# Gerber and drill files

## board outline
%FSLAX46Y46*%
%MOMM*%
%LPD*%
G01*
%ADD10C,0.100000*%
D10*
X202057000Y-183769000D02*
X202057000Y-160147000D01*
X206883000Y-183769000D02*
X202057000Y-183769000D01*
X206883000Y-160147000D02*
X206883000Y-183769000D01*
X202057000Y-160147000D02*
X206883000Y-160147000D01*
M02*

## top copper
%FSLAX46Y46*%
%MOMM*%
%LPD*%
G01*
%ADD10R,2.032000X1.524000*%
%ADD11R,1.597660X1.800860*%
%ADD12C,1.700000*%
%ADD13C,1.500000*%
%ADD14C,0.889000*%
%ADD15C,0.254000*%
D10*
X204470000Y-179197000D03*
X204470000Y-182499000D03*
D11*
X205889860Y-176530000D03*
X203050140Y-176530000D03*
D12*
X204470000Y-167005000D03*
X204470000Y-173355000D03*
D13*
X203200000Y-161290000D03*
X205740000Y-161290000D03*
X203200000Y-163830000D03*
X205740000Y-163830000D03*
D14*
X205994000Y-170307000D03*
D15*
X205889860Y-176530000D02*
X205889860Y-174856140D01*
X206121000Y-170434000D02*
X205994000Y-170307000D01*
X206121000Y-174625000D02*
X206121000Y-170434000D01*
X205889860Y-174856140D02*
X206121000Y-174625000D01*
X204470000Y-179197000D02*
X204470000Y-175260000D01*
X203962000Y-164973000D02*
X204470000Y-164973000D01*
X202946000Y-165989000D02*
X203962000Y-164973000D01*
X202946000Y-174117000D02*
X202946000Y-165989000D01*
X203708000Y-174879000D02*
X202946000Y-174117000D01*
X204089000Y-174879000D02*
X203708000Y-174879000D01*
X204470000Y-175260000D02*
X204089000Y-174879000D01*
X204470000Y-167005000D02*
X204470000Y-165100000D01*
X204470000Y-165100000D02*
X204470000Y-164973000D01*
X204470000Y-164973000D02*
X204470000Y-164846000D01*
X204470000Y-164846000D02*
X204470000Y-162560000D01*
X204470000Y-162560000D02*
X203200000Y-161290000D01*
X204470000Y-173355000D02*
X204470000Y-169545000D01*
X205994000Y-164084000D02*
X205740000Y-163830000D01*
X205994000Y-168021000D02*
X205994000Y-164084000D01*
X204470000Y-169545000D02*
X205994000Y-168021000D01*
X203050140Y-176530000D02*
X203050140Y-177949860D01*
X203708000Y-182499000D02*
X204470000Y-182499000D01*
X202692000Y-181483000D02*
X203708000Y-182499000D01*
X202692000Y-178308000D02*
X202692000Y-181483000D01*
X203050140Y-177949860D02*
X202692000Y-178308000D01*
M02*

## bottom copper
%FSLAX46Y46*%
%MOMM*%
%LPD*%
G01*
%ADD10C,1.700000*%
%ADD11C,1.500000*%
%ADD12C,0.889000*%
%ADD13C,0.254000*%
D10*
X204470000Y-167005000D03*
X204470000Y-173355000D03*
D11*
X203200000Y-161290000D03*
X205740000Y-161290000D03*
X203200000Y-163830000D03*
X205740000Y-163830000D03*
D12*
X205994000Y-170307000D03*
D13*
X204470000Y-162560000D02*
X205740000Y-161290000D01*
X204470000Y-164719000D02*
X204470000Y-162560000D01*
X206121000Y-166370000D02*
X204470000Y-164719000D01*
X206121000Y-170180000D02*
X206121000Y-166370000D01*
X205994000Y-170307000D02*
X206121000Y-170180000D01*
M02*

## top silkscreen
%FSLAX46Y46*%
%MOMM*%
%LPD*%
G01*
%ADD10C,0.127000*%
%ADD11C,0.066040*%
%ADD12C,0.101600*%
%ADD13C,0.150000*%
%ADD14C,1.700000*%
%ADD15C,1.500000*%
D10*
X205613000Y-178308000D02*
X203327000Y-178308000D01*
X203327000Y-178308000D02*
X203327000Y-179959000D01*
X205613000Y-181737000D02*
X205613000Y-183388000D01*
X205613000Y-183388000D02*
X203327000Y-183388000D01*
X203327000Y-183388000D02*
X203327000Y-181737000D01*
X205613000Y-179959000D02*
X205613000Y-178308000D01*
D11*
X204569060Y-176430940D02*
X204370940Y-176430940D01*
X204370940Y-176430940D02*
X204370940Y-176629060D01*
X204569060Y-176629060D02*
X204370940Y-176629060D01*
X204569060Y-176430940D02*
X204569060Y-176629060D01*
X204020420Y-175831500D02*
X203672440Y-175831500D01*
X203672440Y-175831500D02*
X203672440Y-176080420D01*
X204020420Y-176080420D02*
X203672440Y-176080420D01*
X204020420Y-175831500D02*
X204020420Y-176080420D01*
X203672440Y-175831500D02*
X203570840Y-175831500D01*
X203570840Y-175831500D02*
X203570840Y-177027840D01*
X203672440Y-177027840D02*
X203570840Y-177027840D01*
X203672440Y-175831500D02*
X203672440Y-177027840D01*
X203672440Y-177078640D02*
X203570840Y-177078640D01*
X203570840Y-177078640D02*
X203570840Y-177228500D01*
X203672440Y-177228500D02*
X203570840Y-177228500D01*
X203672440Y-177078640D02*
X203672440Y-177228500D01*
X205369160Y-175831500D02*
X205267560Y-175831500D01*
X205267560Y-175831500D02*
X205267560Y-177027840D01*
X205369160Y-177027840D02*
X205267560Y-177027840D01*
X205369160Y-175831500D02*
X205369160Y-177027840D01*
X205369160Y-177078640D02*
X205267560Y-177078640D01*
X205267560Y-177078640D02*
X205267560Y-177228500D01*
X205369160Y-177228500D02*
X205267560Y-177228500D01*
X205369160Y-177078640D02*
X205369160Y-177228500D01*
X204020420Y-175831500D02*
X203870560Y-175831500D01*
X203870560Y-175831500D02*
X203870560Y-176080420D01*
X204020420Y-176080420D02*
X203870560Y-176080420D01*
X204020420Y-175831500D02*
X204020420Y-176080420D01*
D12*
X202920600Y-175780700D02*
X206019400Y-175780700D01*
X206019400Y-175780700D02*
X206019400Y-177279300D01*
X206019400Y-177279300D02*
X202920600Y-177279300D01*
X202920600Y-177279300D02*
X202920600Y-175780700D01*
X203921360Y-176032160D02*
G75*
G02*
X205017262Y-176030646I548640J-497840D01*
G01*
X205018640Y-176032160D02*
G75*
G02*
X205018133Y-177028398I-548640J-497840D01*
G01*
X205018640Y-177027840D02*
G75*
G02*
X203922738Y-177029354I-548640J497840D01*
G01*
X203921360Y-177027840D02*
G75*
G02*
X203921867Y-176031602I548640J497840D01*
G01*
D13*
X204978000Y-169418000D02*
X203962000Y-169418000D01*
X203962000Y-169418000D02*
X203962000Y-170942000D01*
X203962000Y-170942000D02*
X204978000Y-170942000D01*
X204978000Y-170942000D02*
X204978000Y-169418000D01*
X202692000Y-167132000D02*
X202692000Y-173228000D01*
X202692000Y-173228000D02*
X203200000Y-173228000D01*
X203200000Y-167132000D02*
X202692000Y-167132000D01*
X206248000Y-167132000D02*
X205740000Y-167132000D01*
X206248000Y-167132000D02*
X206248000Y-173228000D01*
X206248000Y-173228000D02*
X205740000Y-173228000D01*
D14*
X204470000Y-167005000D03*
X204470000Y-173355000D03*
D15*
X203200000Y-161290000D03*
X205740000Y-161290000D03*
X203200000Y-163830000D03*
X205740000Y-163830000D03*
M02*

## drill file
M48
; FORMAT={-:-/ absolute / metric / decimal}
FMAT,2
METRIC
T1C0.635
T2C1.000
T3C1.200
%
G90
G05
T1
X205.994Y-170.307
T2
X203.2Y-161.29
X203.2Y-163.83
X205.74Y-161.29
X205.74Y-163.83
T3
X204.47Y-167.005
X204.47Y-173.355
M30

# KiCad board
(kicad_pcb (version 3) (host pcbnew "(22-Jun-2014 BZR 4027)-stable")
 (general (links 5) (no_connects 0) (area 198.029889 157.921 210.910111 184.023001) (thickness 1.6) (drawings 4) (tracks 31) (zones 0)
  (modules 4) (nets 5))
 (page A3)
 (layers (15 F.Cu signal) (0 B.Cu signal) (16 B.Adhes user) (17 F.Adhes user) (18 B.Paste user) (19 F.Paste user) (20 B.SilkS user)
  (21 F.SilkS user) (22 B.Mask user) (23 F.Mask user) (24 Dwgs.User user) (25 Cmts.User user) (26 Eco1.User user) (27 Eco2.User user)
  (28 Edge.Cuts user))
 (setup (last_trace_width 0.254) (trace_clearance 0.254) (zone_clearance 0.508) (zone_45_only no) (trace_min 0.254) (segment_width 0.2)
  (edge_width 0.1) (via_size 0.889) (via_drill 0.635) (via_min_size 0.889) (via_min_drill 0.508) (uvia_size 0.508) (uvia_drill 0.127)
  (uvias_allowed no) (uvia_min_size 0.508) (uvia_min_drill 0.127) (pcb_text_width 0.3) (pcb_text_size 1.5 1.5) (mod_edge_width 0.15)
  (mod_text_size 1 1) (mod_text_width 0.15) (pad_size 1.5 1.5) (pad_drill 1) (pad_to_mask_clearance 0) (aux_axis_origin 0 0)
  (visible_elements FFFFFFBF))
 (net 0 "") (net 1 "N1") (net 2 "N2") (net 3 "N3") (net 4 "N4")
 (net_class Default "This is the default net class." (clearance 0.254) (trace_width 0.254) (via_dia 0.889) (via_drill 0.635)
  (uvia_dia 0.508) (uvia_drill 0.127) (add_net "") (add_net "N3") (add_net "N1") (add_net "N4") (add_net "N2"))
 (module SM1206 (layer F.Cu) (at 204.47 180.848 270)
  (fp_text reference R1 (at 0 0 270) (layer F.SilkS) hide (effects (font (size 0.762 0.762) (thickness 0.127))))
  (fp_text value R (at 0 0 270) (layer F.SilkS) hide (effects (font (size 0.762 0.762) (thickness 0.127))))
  (fp_line (start -2.54 -1.143) (end -2.54 1.143) (layer F.SilkS) (width 0.127))
  (fp_line (start -2.54 1.143) (end -0.889 1.143) (layer F.SilkS) (width 0.127))
  (fp_line (start 0.889 -1.143) (end 2.54 -1.143) (layer F.SilkS) (width 0.127))
  (fp_line (start 2.54 -1.143) (end 2.54 1.143) (layer F.SilkS) (width 0.127))
  (fp_line (start 2.54 1.143) (end 0.889 1.143) (layer F.SilkS) (width 0.127))
  (fp_line (start -0.889 -1.143) (end -2.54 -1.143) (layer F.SilkS) (width 0.127))
  (pad 1 smd rect (at -1.651 0 270) (size 1.524 2.032) (layers F.Cu F.Paste F.Mask) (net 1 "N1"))
  (pad 2 smd rect (at 1.651 0 270) (size 1.524 2.032) (layers F.Cu F.Paste F.Mask) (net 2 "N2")))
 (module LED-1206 (layer F.Cu) (at 204.47 176.53 180)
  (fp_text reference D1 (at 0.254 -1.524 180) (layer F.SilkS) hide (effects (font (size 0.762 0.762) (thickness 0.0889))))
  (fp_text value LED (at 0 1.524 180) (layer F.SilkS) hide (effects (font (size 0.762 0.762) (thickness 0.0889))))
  (fp_line (start -0.09906 0.09906) (end 0.09906 0.09906) (layer F.SilkS) (width 0.06604))
  (fp_line (start 0.09906 0.09906) (end 0.09906 -0.09906) (layer F.SilkS) (width 0.06604))
  (fp_line (start -0.09906 -0.09906) (end 0.09906 -0.09906) (layer F.SilkS) (width 0.06604))
  (fp_line (start -0.09906 0.09906) (end -0.09906 -0.09906) (layer F.SilkS) (width 0.06604))
  (fp_line (start 0.44958 0.6985) (end 0.79756 0.6985) (layer F.SilkS) (width 0.06604))
  (fp_line (start 0.79756 0.6985) (end 0.79756 0.44958) (layer F.SilkS) (width 0.06604))
  (fp_line (start 0.44958 0.44958) (end 0.79756 0.44958) (layer F.SilkS) (width 0.06604))
  (fp_line (start 0.44958 0.6985) (end 0.44958 0.44958) (layer F.SilkS) (width 0.06604))
  (fp_line (start 0.79756 0.6985) (end 0.89916 0.6985) (layer F.SilkS) (width 0.06604))
  (fp_line (start 0.89916 0.6985) (end 0.89916 -0.49784) (layer F.SilkS) (width 0.06604))
  (fp_line (start 0.79756 -0.49784) (end 0.89916 -0.49784) (layer F.SilkS) (width 0.06604))
  (fp_line (start 0.79756 0.6985) (end 0.79756 -0.49784) (layer F.SilkS) (width 0.06604))
  (fp_line (start 0.79756 -0.54864) (end 0.89916 -0.54864) (layer F.SilkS) (width 0.06604))
  (fp_line (start 0.89916 -0.54864) (end 0.89916 -0.6985) (layer F.SilkS) (width 0.06604))
  (fp_line (start 0.79756 -0.6985) (end 0.89916 -0.6985) (layer F.SilkS) (width 0.06604))
  (fp_line (start 0.79756 -0.54864) (end 0.79756 -0.6985) (layer F.SilkS) (width 0.06604))
  (fp_line (start -0.89916 0.6985) (end -0.79756 0.6985) (layer F.SilkS) (width 0.06604))
  (fp_line (start -0.79756 0.6985) (end -0.79756 -0.49784) (layer F.SilkS) (width 0.06604))
  (fp_line (start -0.89916 -0.49784) (end -0.79756 -0.49784) (layer F.SilkS) (width 0.06604))
  (fp_line (start -0.89916 0.6985) (end -0.89916 -0.49784) (layer F.SilkS) (width 0.06604))
  (fp_line (start -0.89916 -0.54864) (end -0.79756 -0.54864) (layer F.SilkS) (width 0.06604))
  (fp_line (start -0.79756 -0.54864) (end -0.79756 -0.6985) (layer F.SilkS) (width 0.06604))
  (fp_line (start -0.89916 -0.6985) (end -0.79756 -0.6985) (layer F.SilkS) (width 0.06604))
  (fp_line (start -0.89916 -0.54864) (end -0.89916 -0.6985) (layer F.SilkS) (width 0.06604))
  (fp_line (start 0.44958 0.6985) (end 0.59944 0.6985) (layer F.SilkS) (width 0.06604))
  (fp_line (start 0.59944 0.6985) (end 0.59944 0.44958) (layer F.SilkS) (width 0.06604))
  (fp_line (start 0.44958 0.44958) (end 0.59944 0.44958) (layer F.SilkS) (width 0.06604))
  (fp_line (start 0.44958 0.6985) (end 0.44958 0.44958) (layer F.SilkS) (width 0.06604))
  (fp_line (start 1.5494 0.7493) (end -1.5494 0.7493) (layer F.SilkS) (width 0.1016))
  (fp_line (start -1.5494 0.7493) (end -1.5494 -0.7493) (layer F.SilkS) (width 0.1016))
  (fp_line (start -1.5494 -0.7493) (end 1.5494 -0.7493) (layer F.SilkS) (width 0.1016))
  (fp_line (start 1.5494 -0.7493) (end 1.5494 0.7493) (layer F.SilkS) (width 0.1016))
  (fp_arc (start 0 0) (end 0.54864 0.49784) (angle 95.4) (layer F.SilkS) (width 0.1016))
  (fp_arc (start 0 0) (end -0.54864 0.49784) (angle 84.5) (layer F.SilkS) (width 0.1016))
  (fp_arc (start 0 0) (end -0.54864 -0.49784) (angle 95.4) (layer F.SilkS) (width 0.1016))
  (fp_arc (start 0 0) (end 0.54864 -0.49784) (angle 84.5) (layer F.SilkS) (width 0.1016))
  (pad 1 smd rect (at -1.41986 0 180) (size 1.59766 1.80086) (layers F.Cu F.Paste F.Mask) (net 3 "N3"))
  (pad 2 smd rect (at 1.41986 0 180) (size 1.59766 1.80086) (layers F.Cu F.Paste F.Mask) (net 2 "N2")))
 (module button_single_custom (layer F.Cu) (at 204.47 170.18 270)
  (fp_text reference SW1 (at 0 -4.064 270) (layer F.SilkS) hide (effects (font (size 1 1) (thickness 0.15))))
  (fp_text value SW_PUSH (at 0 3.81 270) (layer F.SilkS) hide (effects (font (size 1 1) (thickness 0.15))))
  (fp_line (start -0.762 -0.508) (end -0.762 0.508) (layer F.SilkS) (width 0.15))
  (fp_line (start -0.762 0.508) (end 0.762 0.508) (layer F.SilkS) (width 0.15))
  (fp_line (start 0.762 0.508) (end 0.762 -0.508) (layer F.SilkS) (width 0.15))
  (fp_line (start 0.762 -0.508) (end -0.762 -0.508) (layer F.SilkS) (width 0.15))
  (fp_line (start -3.048 1.778) (end 3.048 1.778) (layer F.SilkS) (width 0.15))
  (fp_line (start 3.048 1.778) (end 3.048 1.27) (layer F.SilkS) (width 0.15))
  (fp_line (start -3.048 1.27) (end -3.048 1.778) (layer F.SilkS) (width 0.15))
  (fp_line (start -3.048 -1.778) (end -3.048 -1.27) (layer F.SilkS) (width 0.15))
  (fp_line (start -3.048 -1.778) (end 3.048 -1.778) (layer F.SilkS) (width 0.15))
  (fp_line (start 3.048 -1.778) (end 3.048 -1.27) (layer F.SilkS) (width 0.15))
  (pad 1 thru_hole circle (at -3.175 0 270) (size 1.7 1.7) (drill 1.2) (layers *.Cu *.Mask F.SilkS) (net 1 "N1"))
  (pad 2 thru_hole circle (at 3.175 0 270) (size 1.7 1.7) (drill 1.2) (layers *.Cu *.Mask F.SilkS) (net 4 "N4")))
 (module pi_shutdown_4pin (layer F.Cu) (at 204.47 162.56)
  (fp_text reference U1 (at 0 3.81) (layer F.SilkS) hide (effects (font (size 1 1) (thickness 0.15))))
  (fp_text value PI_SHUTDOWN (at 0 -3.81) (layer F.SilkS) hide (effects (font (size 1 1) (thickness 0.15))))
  (pad 14 thru_hole circle (at -1.27 -1.27) (size 1.5 1.5) (drill 1) (layers *.Cu *.Mask F.SilkS) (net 1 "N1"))
  (pad 16 thru_hole circle (at 1.27 -1.27) (size 1.5 1.5) (drill 1) (layers *.Cu *.Mask F.SilkS) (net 3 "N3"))
  (pad 13 thru_hole circle (at -1.27 1.27) (size 1.5 1.5) (drill 1) (layers *.Cu *.Mask F.SilkS))
  (pad 15 thru_hole circle (at 1.27 1.27) (size 1.5 1.5) (drill 1) (layers *.Cu *.Mask F.SilkS) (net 4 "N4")))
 (gr_line (start 202.057 183.769) (end 202.057 160.147) (angle 90) (layer Edge.Cuts) (width 0.1))
 (gr_line (start 206.883 183.769) (end 202.057 183.769) (angle 90) (layer Edge.Cuts) (width 0.1))
 (gr_line (start 206.883 160.147) (end 206.883 183.769) (angle 90) (layer Edge.Cuts) (width 0.1))
 (gr_line (start 202.057 160.147) (end 206.883 160.147) (angle 90) (layer Edge.Cuts) (width 0.1))
 (segment (start 205.88986 176.53) (end 205.88986 174.85614) (width 0.254) (layer F.Cu) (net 3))
 (segment (start 204.47 162.56) (end 205.74 161.29) (width 0.254) (layer B.Cu) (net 3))
 (segment (start 204.47 164.719) (end 204.47 162.56) (width 0.254) (layer B.Cu) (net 3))
 (segment (start 206.121 166.37) (end 204.47 164.719) (width 0.254) (layer B.Cu) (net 3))
 (segment (start 206.121 170.18) (end 206.121 166.37) (width 0.254) (layer B.Cu) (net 3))
 (segment (start 205.994 170.307) (end 206.121 170.18) (width 0.254) (layer B.Cu) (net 3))
 (segment (start 206.121 170.434) (end 205.994 170.307) (width 0.254) (layer F.Cu) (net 3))
 (segment (start 206.121 174.625) (end 206.121 170.434) (width 0.254) (layer F.Cu) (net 3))
 (segment (start 205.88986 174.85614) (end 206.121 174.625) (width 0.254) (layer F.Cu) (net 3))
 (segment (start 204.47 179.197) (end 204.47 175.26) (width 0.254) (layer F.Cu) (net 1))
 (segment (start 203.962 164.973) (end 204.47 164.973) (width 0.254) (layer F.Cu) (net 1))
 (segment (start 202.946 165.989) (end 203.962 164.973) (width 0.254) (layer F.Cu) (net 1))
 (segment (start 202.946 174.117) (end 202.946 165.989) (width 0.254) (layer F.Cu) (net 1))
 (segment (start 203.708 174.879) (end 202.946 174.117) (width 0.254) (layer F.Cu) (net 1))
 (segment (start 204.089 174.879) (end 203.708 174.879) (width 0.254) (layer F.Cu) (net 1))
 (segment (start 204.47 175.26) (end 204.089 174.879) (width 0.254) (layer F.Cu) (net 1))
 (segment (start 204.47 167.005) (end 204.47 165.1) (width 0.254) (layer F.Cu) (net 1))
 (segment (start 204.47 165.1) (end 204.47 164.973) (width 0.254) (layer F.Cu) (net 1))
 (segment (start 204.47 164.973) (end 204.47 164.846) (width 0.254) (layer F.Cu) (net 1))
 (segment (start 204.47 164.846) (end 204.47 162.56) (width 0.254) (layer F.Cu) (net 1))
 (segment (start 204.47 162.56) (end 203.2 161.29) (width 0.254) (layer F.Cu) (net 1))
 (segment (start 204.47 173.355) (end 204.47 169.545) (width 0.254) (layer F.Cu) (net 4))
 (segment (start 205.994 164.084) (end 205.74 163.83) (width 0.254) (layer F.Cu) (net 4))
 (segment (start 205.994 168.021) (end 205.994 164.084) (width 0.254) (layer F.Cu) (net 4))
 (segment (start 204.47 169.545) (end 205.994 168.021) (width 0.254) (layer F.Cu) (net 4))
 (segment (start 203.05014 176.53) (end 203.05014 177.94986) (width 0.254) (layer F.Cu) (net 2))
 (segment (start 203.708 182.499) (end 204.47 182.499) (width 0.254) (layer F.Cu) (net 2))
 (segment (start 202.692 181.483) (end 203.708 182.499) (width 0.254) (layer F.Cu) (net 2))
 (segment (start 202.692 178.308) (end 202.692 181.483) (width 0.254) (layer F.Cu) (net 2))
 (segment (start 203.05014 177.94986) (end 202.692 178.308) (width 0.254) (layer F.Cu) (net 2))
 (via (at 205.994 170.307) (size 0.889) (layers F.Cu B.Cu) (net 3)))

